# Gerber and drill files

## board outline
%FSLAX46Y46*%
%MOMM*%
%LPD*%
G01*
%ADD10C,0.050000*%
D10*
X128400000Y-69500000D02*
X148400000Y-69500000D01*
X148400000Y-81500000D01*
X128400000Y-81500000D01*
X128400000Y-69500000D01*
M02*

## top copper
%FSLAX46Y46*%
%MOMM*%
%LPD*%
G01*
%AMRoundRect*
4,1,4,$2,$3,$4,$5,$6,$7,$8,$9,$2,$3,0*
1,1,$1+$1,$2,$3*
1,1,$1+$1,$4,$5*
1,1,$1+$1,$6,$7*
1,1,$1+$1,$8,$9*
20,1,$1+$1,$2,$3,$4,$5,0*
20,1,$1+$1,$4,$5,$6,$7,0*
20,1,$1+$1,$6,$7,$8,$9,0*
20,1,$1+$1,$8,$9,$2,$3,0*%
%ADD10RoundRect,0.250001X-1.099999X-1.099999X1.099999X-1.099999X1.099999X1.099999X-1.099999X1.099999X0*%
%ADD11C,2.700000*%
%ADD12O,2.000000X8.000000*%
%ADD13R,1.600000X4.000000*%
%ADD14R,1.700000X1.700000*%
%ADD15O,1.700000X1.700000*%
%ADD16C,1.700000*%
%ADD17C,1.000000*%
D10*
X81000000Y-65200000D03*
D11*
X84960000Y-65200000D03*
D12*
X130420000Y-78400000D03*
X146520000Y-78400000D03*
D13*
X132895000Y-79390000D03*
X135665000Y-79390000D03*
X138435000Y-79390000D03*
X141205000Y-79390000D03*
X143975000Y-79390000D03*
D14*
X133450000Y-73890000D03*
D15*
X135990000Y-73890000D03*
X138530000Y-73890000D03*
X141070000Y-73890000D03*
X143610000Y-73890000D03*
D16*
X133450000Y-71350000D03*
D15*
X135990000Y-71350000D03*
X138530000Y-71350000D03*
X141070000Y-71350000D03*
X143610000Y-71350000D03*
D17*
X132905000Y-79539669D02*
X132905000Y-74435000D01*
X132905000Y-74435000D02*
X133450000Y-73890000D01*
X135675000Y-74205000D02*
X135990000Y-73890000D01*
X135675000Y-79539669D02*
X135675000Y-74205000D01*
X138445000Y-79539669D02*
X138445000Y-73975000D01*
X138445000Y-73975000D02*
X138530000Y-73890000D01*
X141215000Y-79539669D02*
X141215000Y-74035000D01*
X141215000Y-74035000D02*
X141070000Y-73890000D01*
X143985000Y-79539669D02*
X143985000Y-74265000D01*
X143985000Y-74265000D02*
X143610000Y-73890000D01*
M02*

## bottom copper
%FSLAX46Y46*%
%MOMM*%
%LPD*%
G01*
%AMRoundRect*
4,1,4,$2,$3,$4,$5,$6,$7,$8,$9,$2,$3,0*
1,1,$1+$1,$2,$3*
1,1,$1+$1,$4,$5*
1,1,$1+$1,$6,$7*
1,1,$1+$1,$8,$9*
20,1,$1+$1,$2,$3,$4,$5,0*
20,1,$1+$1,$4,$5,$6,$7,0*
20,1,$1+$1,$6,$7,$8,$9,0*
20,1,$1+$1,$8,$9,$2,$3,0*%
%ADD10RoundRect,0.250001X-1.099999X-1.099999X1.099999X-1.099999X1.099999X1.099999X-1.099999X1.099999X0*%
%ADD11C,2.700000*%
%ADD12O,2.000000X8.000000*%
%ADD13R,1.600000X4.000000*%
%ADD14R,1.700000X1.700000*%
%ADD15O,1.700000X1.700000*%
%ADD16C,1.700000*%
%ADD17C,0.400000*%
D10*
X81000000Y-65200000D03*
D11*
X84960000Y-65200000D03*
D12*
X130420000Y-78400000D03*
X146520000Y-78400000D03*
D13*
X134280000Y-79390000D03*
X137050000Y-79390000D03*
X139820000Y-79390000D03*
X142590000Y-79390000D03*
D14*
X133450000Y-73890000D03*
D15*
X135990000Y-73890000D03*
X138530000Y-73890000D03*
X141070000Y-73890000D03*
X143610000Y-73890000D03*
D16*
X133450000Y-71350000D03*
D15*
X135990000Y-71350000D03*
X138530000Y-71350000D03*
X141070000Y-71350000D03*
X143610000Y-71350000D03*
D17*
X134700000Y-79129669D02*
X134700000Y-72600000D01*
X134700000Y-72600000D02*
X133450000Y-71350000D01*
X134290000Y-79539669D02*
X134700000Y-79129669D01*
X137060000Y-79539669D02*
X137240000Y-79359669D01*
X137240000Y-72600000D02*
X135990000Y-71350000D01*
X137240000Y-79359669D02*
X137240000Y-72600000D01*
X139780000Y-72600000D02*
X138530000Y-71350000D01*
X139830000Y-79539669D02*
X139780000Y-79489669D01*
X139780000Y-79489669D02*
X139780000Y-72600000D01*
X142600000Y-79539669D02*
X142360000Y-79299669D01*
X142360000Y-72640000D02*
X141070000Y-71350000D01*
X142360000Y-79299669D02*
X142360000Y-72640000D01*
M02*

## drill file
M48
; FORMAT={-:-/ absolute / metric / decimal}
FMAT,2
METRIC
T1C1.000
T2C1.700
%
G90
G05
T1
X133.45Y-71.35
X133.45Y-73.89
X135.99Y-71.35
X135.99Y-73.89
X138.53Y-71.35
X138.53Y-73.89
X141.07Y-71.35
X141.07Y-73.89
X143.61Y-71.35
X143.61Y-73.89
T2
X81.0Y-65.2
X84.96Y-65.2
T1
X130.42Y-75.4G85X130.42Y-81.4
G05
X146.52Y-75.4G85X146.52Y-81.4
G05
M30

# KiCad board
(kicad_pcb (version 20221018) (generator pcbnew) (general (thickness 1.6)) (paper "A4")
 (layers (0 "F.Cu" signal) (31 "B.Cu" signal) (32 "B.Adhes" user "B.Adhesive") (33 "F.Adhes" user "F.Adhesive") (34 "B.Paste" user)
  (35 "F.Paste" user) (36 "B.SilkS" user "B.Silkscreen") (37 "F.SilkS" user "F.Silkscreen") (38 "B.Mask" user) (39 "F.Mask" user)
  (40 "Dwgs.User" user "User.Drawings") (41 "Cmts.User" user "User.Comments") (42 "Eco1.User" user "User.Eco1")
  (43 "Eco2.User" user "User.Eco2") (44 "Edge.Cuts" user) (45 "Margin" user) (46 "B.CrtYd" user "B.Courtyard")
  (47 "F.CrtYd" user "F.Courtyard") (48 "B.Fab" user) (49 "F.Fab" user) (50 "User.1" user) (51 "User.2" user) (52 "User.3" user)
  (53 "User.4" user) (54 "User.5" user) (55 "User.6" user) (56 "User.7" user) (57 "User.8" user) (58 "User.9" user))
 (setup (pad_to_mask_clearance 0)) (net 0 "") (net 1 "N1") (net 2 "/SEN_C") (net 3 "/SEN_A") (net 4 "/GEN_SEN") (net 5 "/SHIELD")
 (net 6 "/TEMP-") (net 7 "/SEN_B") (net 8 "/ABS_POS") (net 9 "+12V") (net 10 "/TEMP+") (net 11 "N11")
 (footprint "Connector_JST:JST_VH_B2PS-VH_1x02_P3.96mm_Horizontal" (layer "F.Cu") (at 81 65.2)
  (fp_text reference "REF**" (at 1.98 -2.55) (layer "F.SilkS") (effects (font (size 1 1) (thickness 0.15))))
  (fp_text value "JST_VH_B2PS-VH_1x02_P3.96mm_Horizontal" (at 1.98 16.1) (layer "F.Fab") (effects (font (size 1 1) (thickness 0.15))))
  (pad "1" thru_hole roundrect (at 0 0) (size 2.7 2.7) (drill 1.7) (layers "*.Cu" "*.Mask") (roundrect_rratio 0.092593))
  (pad "2" thru_hole circle (at 3.96 0) (size 2.7 2.7) (drill 1.7) (layers "*.Cu" "*.Mask")))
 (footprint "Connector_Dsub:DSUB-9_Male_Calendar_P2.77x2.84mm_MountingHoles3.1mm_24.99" (layer "F.Cu") (at 138.4 87)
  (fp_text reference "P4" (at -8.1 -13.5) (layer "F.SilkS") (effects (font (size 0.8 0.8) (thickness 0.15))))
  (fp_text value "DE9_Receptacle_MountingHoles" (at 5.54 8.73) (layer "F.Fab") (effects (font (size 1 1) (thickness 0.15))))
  (pad "0" thru_hole oval (at -7.98 -8.6) (size 2 8) (drill oval 1 7) (layers "*.Cu" "*.Mask") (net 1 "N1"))
  (pad "0" thru_hole oval (at 8.12 -8.6) (size 2 8) (drill oval 1 7) (layers "*.Cu" "*.Mask") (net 1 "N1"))
  (pad "1" smd rect (at -5.505 -7.61) (size 1.6 4) (layers "F.Cu" "F.Paste" "F.Mask") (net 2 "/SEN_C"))
  (pad "2" smd rect (at -2.735 -7.61) (size 1.6 4) (layers "F.Cu" "F.Paste" "F.Mask") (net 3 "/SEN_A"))
  (pad "3" smd rect (at 0.035 -7.61) (size 1.6 4) (layers "F.Cu" "F.Paste" "F.Mask") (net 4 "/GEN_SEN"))
  (pad "4" smd rect (at 2.805 -7.61) (size 1.6 4) (layers "F.Cu" "F.Paste" "F.Mask") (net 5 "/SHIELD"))
  (pad "5" smd rect (at 5.575 -7.61) (size 1.6 4) (layers "F.Cu" "F.Paste" "F.Mask") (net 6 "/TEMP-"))
  (pad "6" smd rect (at -4.12 -7.61) (size 1.6 4) (layers "B.Cu" "B.Paste" "B.Mask") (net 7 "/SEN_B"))
  (pad "7" smd rect (at -1.35 -7.61) (size 1.6 4) (layers "B.Cu" "B.Paste" "B.Mask") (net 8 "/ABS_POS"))
  (pad "8" smd rect (at 1.42 -7.61) (size 1.6 4) (layers "B.Cu" "B.Paste" "B.Mask") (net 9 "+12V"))
  (pad "9" smd rect (at 4.19 -7.61) (size 1.6 4) (layers "B.Cu" "B.Paste" "B.Mask") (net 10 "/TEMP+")))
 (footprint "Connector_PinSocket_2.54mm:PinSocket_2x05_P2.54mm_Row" (layer "F.Cu") (at 133.45 71.35 90)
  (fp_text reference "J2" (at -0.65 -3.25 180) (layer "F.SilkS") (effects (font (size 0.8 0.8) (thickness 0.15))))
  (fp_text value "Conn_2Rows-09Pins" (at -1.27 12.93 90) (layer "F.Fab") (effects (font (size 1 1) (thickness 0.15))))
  (pad "1" thru_hole rect (at -2.54 0 90) (size 1.7 1.7) (drill 1) (layers "*.Cu" "*.Mask") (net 2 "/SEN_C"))
  (pad "2" thru_hole oval (at -2.54 2.54 90) (size 1.7 1.7) (drill 1) (layers "*.Cu" "*.Mask") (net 3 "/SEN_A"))
  (pad "3" thru_hole oval (at -2.54 5.08 90) (size 1.7 1.7) (drill 1) (layers "*.Cu" "*.Mask") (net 4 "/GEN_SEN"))
  (pad "4" thru_hole oval (at -2.54 7.62 90) (size 1.7 1.7) (drill 1) (layers "*.Cu" "*.Mask") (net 5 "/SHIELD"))
  (pad "5" thru_hole oval (at -2.54 10.16 90) (size 1.7 1.7) (drill 1) (layers "*.Cu" "*.Mask") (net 6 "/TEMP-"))
  (pad "6" thru_hole circle (at 0 0 90) (size 1.7 1.7) (drill 1) (layers "*.Cu" "*.Mask") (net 7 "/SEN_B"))
  (pad "7" thru_hole oval (at 0 2.54 90) (size 1.7 1.7) (drill 1) (layers "*.Cu" "*.Mask") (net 8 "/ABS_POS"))
  (pad "8" thru_hole oval (at 0 5.08 90) (size 1.7 1.7) (drill 1) (layers "*.Cu" "*.Mask") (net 9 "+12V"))
  (pad "9" thru_hole oval (at 0 7.62 90) (size 1.7 1.7) (drill 1) (layers "*.Cu" "*.Mask") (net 10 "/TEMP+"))
  (pad "10" thru_hole oval (at 0 10.16 90) (size 1.7 1.7) (drill 1) (layers "*.Cu" "*.Mask") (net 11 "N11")))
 (gr_rect (start 128.4 69.5) (end 148.4 81.5) (stroke (width 0.05) (type default)) (fill none) (layer "Edge.Cuts"))
 (segment (start 132.905 79.539669) (end 132.905 74.435) (width 1) (layer "F.Cu") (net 2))
 (segment (start 132.905 74.435) (end 133.45 73.89) (width 1) (layer "F.Cu") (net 2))
 (segment (start 135.675 74.205) (end 135.99 73.89) (width 1) (layer "F.Cu") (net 3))
 (segment (start 135.675 79.539669) (end 135.675 74.205) (width 1) (layer "F.Cu") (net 3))
 (segment (start 138.445 79.539669) (end 138.445 73.975) (width 1) (layer "F.Cu") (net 4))
 (segment (start 138.445 73.975) (end 138.53 73.89) (width 1) (layer "F.Cu") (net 4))
 (segment (start 141.215 79.539669) (end 141.215 74.035) (width 1) (layer "F.Cu") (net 5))
 (segment (start 141.215 74.035) (end 141.07 73.89) (width 1) (layer "F.Cu") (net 5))
 (segment (start 143.985 79.539669) (end 143.985 74.265) (width 1) (layer "F.Cu") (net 6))
 (segment (start 143.985 74.265) (end 143.61 73.89) (width 1) (layer "F.Cu") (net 6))
 (segment (start 134.7 79.129669) (end 134.7 72.6) (width 0.4) (layer "B.Cu") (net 7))
 (segment (start 134.7 72.6) (end 133.45 71.35) (width 0.4) (layer "B.Cu") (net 7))
 (segment (start 134.29 79.539669) (end 134.7 79.129669) (width 0.4) (layer "B.Cu") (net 7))
 (segment (start 137.06 79.539669) (end 137.24 79.359669) (width 0.4) (layer "B.Cu") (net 8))
 (segment (start 137.24 72.6) (end 135.99 71.35) (width 0.4) (layer "B.Cu") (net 8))
 (segment (start 137.24 79.359669) (end 137.24 72.6) (width 0.4) (layer "B.Cu") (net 8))
 (segment (start 139.78 72.6) (end 138.53 71.35) (width 0.4) (layer "B.Cu") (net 9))
 (segment (start 139.83 79.539669) (end 139.78 79.489669) (width 0.4) (layer "B.Cu") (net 9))
 (segment (start 139.78 79.489669) (end 139.78 72.6) (width 0.4) (layer "B.Cu") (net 9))
 (segment (start 142.6 79.539669) (end 142.36 79.299669) (width 0.4) (layer "B.Cu") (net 10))
 (segment (start 142.36 72.64) (end 141.07 71.35) (width 0.4) (layer "B.Cu") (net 10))
 (segment (start 142.36 79.299669) (end 142.36 72.64) (width 0.4) (layer "B.Cu") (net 10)))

